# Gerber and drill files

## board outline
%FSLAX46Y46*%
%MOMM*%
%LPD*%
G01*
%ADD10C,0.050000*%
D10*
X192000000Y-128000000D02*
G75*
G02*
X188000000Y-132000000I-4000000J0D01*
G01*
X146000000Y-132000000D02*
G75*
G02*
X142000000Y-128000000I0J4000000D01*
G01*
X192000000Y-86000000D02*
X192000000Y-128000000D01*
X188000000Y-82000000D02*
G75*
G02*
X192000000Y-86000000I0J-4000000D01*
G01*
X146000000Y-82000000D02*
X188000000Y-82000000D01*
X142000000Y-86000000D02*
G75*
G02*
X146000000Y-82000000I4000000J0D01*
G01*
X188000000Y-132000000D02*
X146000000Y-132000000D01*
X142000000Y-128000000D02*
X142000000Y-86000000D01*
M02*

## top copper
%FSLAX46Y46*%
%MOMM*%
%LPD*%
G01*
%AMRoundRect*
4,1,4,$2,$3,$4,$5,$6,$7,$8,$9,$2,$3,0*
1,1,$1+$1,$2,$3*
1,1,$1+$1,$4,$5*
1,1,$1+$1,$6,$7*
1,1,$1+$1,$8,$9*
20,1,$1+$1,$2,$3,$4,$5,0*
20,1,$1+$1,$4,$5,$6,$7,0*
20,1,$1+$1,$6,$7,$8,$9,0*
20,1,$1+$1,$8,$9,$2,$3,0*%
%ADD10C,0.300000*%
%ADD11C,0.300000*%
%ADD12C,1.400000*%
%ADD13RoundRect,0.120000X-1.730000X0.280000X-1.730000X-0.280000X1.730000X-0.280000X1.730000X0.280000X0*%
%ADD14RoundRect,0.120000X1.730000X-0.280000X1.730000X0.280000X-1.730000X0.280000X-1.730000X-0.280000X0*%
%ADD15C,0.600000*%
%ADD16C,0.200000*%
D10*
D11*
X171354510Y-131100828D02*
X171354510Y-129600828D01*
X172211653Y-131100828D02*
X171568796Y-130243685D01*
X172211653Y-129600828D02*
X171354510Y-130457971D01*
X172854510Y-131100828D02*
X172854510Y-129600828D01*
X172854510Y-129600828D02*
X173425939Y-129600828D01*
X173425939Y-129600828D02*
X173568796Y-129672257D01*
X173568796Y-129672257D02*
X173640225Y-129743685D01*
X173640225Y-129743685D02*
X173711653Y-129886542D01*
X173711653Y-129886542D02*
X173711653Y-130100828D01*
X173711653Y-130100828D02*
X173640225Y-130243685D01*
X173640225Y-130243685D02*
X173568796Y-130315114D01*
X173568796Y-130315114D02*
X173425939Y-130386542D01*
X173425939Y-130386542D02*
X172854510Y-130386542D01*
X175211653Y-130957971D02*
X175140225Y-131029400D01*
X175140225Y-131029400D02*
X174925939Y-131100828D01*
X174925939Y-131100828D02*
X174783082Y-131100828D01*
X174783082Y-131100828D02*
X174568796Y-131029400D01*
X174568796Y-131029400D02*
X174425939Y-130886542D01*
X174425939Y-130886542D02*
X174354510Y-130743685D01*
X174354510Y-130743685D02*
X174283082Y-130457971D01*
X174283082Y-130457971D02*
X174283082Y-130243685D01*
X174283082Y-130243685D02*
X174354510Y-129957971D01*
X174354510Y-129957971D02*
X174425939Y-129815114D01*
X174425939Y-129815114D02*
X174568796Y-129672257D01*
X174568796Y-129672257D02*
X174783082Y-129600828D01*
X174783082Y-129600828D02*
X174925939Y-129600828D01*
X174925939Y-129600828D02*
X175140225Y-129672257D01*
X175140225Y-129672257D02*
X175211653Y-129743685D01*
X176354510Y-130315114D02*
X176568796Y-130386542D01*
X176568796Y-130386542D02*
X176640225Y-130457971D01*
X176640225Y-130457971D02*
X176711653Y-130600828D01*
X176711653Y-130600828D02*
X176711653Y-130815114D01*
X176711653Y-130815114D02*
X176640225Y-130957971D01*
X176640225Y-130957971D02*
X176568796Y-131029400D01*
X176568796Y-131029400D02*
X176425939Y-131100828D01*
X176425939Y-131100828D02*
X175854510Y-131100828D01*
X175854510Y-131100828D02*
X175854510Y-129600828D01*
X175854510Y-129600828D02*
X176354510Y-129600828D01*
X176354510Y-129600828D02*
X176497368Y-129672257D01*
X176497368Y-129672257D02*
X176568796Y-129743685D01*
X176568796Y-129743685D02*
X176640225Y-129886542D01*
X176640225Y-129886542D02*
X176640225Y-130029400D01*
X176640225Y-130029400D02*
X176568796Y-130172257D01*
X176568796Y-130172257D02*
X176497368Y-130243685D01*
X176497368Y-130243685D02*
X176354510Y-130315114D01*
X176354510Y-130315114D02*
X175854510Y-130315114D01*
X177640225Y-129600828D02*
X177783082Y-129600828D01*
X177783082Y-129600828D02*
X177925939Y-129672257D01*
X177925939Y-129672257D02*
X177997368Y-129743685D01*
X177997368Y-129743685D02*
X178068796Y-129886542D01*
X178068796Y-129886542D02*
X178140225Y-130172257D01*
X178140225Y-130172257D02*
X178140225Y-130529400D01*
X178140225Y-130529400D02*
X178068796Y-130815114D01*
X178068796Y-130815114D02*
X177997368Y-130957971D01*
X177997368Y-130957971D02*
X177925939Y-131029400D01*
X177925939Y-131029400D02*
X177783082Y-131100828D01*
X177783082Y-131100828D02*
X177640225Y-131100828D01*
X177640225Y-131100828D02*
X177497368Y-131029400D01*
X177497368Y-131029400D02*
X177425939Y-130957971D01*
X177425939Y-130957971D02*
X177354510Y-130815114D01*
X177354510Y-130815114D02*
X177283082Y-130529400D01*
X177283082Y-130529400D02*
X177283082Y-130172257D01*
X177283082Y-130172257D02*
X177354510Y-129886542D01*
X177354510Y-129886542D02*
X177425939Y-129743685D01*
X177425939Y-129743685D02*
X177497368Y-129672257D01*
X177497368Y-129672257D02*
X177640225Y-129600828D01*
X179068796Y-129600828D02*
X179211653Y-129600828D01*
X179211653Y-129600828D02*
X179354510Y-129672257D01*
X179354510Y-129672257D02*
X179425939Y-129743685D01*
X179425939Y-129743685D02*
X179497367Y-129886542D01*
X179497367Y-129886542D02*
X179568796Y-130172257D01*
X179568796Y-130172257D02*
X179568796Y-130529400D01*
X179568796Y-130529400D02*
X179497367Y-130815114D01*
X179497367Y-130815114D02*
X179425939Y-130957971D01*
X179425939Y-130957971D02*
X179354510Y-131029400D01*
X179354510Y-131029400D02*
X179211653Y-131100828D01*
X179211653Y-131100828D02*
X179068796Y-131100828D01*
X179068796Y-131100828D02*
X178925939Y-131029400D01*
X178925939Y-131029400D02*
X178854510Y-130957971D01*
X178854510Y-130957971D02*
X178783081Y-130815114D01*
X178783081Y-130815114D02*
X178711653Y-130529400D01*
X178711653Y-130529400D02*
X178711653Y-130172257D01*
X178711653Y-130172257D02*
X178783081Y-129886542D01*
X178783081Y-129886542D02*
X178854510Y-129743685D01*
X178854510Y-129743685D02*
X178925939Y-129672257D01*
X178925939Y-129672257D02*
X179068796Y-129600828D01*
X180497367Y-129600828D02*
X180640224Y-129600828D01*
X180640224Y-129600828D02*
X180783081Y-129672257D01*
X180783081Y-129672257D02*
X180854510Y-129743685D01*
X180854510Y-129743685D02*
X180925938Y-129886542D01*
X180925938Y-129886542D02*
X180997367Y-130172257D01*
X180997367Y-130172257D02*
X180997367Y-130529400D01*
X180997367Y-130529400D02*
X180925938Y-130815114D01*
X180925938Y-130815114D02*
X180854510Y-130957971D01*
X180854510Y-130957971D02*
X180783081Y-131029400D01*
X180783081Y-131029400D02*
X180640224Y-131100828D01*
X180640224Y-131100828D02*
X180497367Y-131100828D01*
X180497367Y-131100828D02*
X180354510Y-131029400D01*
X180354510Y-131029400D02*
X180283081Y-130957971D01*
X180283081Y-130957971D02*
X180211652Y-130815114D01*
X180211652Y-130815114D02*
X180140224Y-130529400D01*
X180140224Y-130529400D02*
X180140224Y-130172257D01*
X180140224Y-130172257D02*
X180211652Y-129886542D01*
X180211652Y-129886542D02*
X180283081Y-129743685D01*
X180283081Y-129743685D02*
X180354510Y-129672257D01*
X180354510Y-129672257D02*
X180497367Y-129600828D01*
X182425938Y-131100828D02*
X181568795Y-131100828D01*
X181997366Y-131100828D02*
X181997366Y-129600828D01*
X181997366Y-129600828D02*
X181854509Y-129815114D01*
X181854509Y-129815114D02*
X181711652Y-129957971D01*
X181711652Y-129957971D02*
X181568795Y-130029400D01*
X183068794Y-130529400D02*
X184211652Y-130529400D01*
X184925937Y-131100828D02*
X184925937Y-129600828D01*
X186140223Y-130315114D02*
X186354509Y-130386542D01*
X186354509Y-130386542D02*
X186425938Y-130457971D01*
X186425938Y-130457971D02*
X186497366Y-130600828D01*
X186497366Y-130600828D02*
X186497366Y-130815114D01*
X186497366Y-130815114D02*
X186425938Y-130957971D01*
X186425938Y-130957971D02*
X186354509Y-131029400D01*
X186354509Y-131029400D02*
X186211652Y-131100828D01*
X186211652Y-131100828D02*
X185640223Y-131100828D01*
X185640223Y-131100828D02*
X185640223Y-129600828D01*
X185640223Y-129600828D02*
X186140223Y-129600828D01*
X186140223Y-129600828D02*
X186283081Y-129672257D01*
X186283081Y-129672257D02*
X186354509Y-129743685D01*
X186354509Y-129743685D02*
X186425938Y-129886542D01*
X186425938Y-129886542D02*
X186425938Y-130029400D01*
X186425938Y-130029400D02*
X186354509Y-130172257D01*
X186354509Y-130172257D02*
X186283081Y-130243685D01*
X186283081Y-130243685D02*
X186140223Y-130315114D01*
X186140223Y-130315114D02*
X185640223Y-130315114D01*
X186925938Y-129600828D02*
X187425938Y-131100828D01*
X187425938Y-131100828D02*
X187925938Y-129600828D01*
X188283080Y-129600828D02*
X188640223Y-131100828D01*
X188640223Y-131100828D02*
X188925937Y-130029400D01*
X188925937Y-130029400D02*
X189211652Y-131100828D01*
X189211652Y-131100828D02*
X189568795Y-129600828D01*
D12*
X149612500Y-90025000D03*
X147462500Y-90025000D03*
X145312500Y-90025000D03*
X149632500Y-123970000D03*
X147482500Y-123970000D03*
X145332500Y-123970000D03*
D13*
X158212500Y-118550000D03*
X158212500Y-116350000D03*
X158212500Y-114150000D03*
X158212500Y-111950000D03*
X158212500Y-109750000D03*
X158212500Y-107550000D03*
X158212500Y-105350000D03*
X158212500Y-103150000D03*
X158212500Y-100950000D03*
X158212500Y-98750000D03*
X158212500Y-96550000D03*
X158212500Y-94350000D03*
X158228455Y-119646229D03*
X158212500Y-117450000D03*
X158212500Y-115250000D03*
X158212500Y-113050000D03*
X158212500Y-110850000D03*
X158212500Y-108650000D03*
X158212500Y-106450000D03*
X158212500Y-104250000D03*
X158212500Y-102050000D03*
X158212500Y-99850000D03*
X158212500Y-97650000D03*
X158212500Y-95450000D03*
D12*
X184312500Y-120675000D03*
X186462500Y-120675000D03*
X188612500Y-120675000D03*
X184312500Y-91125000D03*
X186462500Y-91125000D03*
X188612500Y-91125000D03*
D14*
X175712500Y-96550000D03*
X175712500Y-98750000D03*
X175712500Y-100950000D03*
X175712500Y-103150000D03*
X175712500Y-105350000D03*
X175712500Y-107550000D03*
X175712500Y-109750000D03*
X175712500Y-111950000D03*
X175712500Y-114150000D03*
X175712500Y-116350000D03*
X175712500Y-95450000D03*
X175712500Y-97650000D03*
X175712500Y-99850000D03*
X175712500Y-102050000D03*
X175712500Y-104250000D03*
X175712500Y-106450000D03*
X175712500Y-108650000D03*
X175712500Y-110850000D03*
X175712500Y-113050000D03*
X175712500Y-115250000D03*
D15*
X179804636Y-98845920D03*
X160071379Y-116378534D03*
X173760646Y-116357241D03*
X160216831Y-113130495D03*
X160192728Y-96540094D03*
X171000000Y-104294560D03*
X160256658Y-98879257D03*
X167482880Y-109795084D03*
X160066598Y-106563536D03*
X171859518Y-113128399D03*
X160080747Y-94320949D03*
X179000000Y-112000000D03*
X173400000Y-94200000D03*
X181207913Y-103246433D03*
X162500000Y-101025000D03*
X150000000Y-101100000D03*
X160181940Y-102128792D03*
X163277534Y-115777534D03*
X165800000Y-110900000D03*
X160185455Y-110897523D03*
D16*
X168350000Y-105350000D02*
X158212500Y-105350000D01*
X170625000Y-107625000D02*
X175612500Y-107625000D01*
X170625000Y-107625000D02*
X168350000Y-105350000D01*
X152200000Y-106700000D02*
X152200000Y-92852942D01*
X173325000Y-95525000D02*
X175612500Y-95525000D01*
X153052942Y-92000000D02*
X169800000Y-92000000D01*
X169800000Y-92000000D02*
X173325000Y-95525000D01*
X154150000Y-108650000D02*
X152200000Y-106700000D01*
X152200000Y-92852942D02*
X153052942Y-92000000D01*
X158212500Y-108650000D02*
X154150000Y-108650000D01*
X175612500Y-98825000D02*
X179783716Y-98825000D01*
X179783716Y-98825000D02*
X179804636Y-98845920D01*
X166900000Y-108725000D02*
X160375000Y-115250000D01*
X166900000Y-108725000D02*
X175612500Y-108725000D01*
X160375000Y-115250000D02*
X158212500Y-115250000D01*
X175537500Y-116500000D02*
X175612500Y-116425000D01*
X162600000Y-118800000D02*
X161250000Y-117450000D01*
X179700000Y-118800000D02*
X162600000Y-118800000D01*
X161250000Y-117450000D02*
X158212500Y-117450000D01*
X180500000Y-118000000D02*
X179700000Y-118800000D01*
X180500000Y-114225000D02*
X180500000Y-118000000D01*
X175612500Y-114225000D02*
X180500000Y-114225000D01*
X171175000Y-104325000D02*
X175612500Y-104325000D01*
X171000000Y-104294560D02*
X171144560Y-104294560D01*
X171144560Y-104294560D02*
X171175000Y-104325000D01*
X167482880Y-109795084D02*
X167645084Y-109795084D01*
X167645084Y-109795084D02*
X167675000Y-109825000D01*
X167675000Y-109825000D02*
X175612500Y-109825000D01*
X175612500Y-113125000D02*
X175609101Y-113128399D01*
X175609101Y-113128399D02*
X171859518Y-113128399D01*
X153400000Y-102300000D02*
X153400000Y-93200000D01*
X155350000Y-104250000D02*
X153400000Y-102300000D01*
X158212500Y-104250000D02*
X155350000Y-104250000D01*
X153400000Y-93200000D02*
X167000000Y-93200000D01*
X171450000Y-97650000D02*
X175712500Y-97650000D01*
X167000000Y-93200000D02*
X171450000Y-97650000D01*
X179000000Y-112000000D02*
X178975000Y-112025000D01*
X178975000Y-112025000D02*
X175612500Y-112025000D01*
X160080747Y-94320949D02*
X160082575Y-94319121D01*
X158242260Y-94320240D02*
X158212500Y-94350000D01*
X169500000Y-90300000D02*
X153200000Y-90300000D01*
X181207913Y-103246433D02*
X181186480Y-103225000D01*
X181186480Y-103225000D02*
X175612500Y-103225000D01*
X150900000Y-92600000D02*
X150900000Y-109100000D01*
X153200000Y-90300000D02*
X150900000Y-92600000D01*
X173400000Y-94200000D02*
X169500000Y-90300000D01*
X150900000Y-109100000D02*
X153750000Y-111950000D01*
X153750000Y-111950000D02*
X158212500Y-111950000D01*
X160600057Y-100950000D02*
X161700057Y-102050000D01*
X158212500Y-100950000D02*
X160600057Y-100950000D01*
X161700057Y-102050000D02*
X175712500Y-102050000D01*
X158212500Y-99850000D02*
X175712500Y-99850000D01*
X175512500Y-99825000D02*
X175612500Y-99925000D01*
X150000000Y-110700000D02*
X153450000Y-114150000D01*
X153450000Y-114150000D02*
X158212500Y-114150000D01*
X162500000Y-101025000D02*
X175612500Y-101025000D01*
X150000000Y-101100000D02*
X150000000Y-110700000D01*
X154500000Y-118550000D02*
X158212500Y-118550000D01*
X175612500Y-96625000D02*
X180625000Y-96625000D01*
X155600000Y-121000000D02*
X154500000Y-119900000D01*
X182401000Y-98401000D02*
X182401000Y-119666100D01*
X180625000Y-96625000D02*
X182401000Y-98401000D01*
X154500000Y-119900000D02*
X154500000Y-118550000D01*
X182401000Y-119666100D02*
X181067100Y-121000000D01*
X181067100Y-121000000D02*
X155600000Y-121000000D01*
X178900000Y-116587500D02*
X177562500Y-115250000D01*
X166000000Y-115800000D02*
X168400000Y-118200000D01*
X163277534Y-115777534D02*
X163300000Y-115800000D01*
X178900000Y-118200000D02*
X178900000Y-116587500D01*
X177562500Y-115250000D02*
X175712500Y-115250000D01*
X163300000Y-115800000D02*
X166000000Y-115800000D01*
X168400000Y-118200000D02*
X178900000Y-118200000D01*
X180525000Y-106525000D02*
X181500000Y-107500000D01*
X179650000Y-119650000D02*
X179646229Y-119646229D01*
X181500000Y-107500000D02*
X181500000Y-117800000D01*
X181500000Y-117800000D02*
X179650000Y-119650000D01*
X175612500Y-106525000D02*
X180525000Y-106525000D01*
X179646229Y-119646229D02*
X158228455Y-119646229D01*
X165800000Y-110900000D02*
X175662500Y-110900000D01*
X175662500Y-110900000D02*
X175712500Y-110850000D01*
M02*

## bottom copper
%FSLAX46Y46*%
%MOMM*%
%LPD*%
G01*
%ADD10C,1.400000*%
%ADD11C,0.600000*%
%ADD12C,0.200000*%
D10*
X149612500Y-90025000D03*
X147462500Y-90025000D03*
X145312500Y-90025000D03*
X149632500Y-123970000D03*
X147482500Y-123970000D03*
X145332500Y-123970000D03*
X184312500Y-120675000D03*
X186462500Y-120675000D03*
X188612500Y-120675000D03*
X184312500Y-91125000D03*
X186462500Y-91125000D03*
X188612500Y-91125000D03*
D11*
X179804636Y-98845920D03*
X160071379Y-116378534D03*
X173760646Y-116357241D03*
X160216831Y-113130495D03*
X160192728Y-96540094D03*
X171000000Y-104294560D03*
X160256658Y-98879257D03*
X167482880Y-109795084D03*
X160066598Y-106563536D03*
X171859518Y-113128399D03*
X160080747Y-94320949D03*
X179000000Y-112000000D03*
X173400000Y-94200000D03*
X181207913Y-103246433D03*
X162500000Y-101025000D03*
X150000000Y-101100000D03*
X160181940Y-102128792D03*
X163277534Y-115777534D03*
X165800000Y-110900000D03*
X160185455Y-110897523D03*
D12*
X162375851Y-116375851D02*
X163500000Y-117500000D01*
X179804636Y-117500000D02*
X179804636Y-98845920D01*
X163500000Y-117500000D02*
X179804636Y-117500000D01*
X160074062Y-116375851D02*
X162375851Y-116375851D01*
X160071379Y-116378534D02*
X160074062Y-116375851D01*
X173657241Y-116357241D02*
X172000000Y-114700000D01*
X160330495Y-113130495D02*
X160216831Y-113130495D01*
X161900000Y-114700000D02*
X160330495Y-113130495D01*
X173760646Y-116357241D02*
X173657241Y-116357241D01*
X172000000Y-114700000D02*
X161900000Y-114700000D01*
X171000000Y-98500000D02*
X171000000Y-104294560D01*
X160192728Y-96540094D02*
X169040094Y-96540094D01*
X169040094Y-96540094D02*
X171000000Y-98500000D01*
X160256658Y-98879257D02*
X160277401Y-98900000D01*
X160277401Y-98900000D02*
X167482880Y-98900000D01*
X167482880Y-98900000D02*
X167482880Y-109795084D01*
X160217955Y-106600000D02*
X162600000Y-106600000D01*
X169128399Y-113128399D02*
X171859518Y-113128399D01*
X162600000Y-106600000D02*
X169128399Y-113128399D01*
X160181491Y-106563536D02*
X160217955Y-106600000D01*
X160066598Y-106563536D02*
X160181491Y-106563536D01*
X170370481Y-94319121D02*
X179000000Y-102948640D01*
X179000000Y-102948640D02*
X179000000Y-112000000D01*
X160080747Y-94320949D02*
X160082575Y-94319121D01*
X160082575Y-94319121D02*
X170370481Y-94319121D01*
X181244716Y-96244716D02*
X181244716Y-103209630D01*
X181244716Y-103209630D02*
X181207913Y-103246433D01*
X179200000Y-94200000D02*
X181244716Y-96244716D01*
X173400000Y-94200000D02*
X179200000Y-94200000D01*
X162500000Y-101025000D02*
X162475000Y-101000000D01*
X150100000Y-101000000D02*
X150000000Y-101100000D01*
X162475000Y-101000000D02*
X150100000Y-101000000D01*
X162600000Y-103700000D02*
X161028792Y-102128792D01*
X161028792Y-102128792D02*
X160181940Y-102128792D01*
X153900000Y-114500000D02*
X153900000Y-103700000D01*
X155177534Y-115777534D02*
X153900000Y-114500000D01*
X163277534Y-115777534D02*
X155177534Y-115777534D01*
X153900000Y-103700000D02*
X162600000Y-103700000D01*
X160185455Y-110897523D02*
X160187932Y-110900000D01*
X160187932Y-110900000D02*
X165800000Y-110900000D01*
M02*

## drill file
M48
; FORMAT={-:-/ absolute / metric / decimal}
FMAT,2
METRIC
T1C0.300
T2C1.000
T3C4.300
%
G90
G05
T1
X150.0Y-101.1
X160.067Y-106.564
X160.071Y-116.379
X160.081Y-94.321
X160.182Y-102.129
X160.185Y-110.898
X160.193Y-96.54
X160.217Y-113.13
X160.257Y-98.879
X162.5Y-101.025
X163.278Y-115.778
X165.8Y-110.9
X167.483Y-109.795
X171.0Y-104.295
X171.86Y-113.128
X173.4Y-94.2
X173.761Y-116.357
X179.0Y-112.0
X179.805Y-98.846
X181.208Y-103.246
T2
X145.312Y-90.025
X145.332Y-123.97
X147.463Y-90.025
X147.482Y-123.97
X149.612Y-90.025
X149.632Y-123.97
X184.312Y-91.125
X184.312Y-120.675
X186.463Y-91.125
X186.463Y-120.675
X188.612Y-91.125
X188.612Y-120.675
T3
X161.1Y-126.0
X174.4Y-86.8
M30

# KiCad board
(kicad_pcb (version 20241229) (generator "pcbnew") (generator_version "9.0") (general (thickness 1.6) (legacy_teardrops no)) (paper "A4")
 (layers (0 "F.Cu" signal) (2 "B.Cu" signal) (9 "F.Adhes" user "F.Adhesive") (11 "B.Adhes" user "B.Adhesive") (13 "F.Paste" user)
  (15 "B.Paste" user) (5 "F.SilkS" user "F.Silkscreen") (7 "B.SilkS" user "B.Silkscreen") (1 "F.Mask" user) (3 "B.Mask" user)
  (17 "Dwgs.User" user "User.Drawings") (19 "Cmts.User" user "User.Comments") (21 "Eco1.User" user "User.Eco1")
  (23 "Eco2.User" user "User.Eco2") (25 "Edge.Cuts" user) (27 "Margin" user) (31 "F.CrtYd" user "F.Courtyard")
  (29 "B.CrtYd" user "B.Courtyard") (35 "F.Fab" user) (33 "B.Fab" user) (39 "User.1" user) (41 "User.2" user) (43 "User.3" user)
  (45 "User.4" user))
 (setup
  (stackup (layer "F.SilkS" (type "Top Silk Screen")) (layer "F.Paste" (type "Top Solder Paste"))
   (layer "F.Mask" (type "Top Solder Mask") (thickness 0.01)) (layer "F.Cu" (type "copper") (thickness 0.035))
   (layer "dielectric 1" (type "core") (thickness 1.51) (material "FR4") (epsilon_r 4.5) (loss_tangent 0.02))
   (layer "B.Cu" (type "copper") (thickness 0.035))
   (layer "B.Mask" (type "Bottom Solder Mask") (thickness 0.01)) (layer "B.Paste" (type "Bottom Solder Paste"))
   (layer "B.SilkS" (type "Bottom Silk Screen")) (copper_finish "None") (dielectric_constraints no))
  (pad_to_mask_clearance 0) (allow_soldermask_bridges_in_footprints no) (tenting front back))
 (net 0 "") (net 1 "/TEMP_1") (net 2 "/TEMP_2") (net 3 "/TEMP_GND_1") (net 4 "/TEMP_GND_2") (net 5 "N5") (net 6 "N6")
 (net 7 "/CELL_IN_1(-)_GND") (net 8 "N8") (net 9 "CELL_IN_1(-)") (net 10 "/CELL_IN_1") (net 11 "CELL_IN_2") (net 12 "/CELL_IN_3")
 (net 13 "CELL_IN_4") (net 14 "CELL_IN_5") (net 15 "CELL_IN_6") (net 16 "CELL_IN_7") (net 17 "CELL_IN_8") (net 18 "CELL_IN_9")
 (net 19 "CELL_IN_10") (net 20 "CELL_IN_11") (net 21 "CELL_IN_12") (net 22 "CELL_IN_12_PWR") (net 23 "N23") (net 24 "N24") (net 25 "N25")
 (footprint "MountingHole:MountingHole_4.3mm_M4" (layer "F.Cu") (at 174.4 86.8)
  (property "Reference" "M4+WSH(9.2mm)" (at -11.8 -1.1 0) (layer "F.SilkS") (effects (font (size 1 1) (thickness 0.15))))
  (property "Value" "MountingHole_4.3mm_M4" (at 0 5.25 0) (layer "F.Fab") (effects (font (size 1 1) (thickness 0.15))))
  (pad "" np_thru_hole circle (at 0 0) (size 4.3 4.3) (drill 4.3) (layers "*.Cu" "*.Mask")))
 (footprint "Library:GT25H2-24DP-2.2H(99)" (layer "F.Cu") (at 160.4625 107 -90)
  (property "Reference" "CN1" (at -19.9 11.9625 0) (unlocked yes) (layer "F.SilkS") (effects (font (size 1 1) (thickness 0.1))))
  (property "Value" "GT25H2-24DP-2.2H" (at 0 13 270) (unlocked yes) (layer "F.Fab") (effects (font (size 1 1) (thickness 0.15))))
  (pad "" np_thru_hole circle (at -16.975 10.85 270) (size 1.4 1.4) (drill 1) (layers "*.Cu" "*.Mask"))
  (pad "" np_thru_hole circle (at -16.975 13 270) (size 1.4 1.4) (drill 1) (layers "*.Cu" "*.Mask"))
  (pad "" np_thru_hole circle (at -16.975 15.15 270) (size 1.4 1.4) (drill 1) (layers "*.Cu" "*.Mask"))
  (pad "" np_thru_hole circle (at 16.97 10.83 270) (size 1.4 1.4) (drill 1) (layers "*.Cu" "*.Mask"))
  (pad "" np_thru_hole circle (at 16.97 12.98 270) (size 1.4 1.4) (drill 1) (layers "*.Cu" "*.Mask"))
  (pad "" np_thru_hole circle (at 16.97 15.13 270) (size 1.4 1.4) (drill 1) (layers "*.Cu" "*.Mask"))
  (pad "1" smd roundrect (at 11.55 2.25 270) (size 0.8 3.7) (layers "F.Cu" "F.Mask" "F.Paste") (roundrect_rratio 0.15) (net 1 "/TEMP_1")
   (thermal_bridge_angle 45))
  (pad "2" smd roundrect (at 9.35 2.25 270) (size 0.8 3.7) (layers "F.Cu" "F.Mask" "F.Paste") (roundrect_rratio 0.15) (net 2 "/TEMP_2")
   (thermal_bridge_angle 45))
  (pad "3" smd roundrect (at 7.15 2.25 270) (size 0.8 3.7) (layers "F.Cu" "F.Mask" "F.Paste") (roundrect_rratio 0.15) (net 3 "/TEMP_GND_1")
   (thermal_bridge_angle 45))
  (pad "4" smd roundrect (at 4.95 2.25 270) (size 0.8 3.7) (layers "F.Cu" "F.Mask" "F.Paste") (roundrect_rratio 0.15) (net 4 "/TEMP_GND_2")
   (thermal_bridge_angle 45))
  (pad "5" smd roundrect (at 2.75 2.25 270) (size 0.8 3.7) (layers "F.Cu" "F.Mask" "F.Paste") (roundrect_rratio 0.15) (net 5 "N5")
   (thermal_bridge_angle 45))
  (pad "6" smd roundrect (at 0.55 2.25 270) (size 0.8 3.7) (layers "F.Cu" "F.Mask" "F.Paste") (roundrect_rratio 0.15) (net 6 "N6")
   (thermal_bridge_angle 45))
  (pad "7" smd roundrect (at -1.65 2.25 270) (size 0.8 3.7) (layers "F.Cu" "F.Mask" "F.Paste") (roundrect_rratio 0.15)
   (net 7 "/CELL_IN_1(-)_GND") (thermal_bridge_angle 45))
  (pad "8" smd roundrect (at -3.85 2.25 270) (size 0.8 3.7) (layers "F.Cu" "F.Mask" "F.Paste") (roundrect_rratio 0.15) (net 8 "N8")
   (thermal_bridge_angle 45))
  (pad "9" smd roundrect (at -6.05 2.25 270) (size 0.8 3.7) (layers "F.Cu" "F.Mask" "F.Paste") (roundrect_rratio 0.15)
   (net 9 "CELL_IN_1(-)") (thermal_bridge_angle 45))
  (pad "10" smd roundrect (at -8.25 2.25 270) (size 0.8 3.7) (layers "F.Cu" "F.Mask" "F.Paste") (roundrect_rratio 0.15)
   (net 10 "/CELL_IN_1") (thermal_bridge_angle 45))
  (pad "11" smd roundrect (at -10.45 2.25 270) (size 0.8 3.7) (layers "F.Cu" "F.Mask" "F.Paste") (roundrect_rratio 0.15)
   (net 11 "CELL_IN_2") (thermal_bridge_angle 45))
  (pad "12" smd roundrect (at -12.65 2.25 270) (size 0.8 3.7) (layers "F.Cu" "F.Mask" "F.Paste") (roundrect_rratio 0.15)
   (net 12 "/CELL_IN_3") (thermal_bridge_angle 45))
  (pad "13" smd roundrect (at 12.646229 2.234045 270) (size 0.8 3.7) (layers "F.Cu" "F.Mask" "F.Paste") (roundrect_rratio 0.15)
   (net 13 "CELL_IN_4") (thermal_bridge_angle 45))
  (pad "14" smd roundrect (at 10.45 2.25 270) (size 0.8 3.7) (layers "F.Cu" "F.Mask" "F.Paste") (roundrect_rratio 0.15) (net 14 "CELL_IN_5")
   (thermal_bridge_angle 45))
  (pad "15" smd roundrect (at 8.25 2.25 270) (size 0.8 3.7) (layers "F.Cu" "F.Mask" "F.Paste") (roundrect_rratio 0.15) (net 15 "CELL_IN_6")
   (thermal_bridge_angle 45))
  (pad "16" smd roundrect (at 6.05 2.25 270) (size 0.8 3.7) (layers "F.Cu" "F.Mask" "F.Paste") (roundrect_rratio 0.15) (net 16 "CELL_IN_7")
   (thermal_bridge_angle 45))
  (pad "17" smd roundrect (at 3.85 2.25 270) (size 0.8 3.7) (layers "F.Cu" "F.Mask" "F.Paste") (roundrect_rratio 0.15) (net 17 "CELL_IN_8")
   (thermal_bridge_angle 45))
  (pad "18" smd roundrect (at 1.65 2.25 270) (size 0.8 3.7) (layers "F.Cu" "F.Mask" "F.Paste") (roundrect_rratio 0.15) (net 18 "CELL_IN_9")
   (thermal_bridge_angle 45))
  (pad "19" smd roundrect (at -0.55 2.25 270) (size 0.8 3.7) (layers "F.Cu" "F.Mask" "F.Paste") (roundrect_rratio 0.15)
   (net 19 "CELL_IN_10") (thermal_bridge_angle 45))
  (pad "20" smd roundrect (at -2.75 2.25 270) (size 0.8 3.7) (layers "F.Cu" "F.Mask" "F.Paste") (roundrect_rratio 0.15)
   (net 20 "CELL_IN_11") (thermal_bridge_angle 45))
  (pad "21" smd roundrect (at -4.95 2.25 270) (size 0.8 3.7) (layers "F.Cu" "F.Mask" "F.Paste") (roundrect_rratio 0.15)
   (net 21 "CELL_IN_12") (thermal_bridge_angle 45))
  (pad "22" smd roundrect (at -7.15 2.25 270) (size 0.8 3.7) (layers "F.Cu" "F.Mask" "F.Paste") (roundrect_rratio 0.15)
   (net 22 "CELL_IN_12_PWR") (thermal_bridge_angle 45))
  (pad "23" smd roundrect (at -9.35 2.25 270) (size 0.8 3.7) (layers "F.Cu" "F.Mask" "F.Paste") (roundrect_rratio 0.15) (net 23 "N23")
   (thermal_bridge_angle 45))
  (pad "24" smd roundrect (at -11.55 2.25 270) (size 0.8 3.7) (layers "F.Cu" "F.Mask" "F.Paste") (roundrect_rratio 0.15) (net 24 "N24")
   (thermal_bridge_angle 45)))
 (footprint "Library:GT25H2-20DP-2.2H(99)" (layer "F.Cu") (at 173.4625 105.9 90)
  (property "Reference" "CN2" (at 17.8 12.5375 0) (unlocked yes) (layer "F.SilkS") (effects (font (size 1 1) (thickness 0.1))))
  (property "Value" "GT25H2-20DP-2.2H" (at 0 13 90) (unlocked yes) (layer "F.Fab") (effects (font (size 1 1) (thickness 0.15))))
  (pad "" np_thru_hole circle (at -14.775 10.85 90) (size 1.4 1.4) (drill 1) (layers "*.Cu" "*.Mask"))
  (pad "" np_thru_hole circle (at -14.775 13 90) (size 1.4 1.4) (drill 1) (layers "*.Cu" "*.Mask"))
  (pad "" np_thru_hole circle (at -14.775 15.15 90) (size 1.4 1.4) (drill 1) (layers "*.Cu" "*.Mask"))
  (pad "" np_thru_hole circle (at 14.775 10.85 90) (size 1.4 1.4) (drill 1) (layers "*.Cu" "*.Mask"))
  (pad "" np_thru_hole circle (at 14.775 13 90) (size 1.4 1.4) (drill 1) (layers "*.Cu" "*.Mask"))
  (pad "" np_thru_hole circle (at 14.775 15.15 90) (size 1.4 1.4) (drill 1) (layers "*.Cu" "*.Mask"))
  (pad "1" smd roundrect (at 9.35 2.25 90) (size 0.8 3.7) (layers "F.Cu" "F.Mask" "F.Paste") (roundrect_rratio 0.15) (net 1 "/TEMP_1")
   (thermal_bridge_angle 45))
  (pad "2" smd roundrect (at 7.15 2.25 90) (size 0.8 3.7) (layers "F.Cu" "F.Mask" "F.Paste") (roundrect_rratio 0.15) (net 2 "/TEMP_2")
   (thermal_bridge_angle 45))
  (pad "3" smd roundrect (at 4.95 2.25 90) (size 0.8 3.7) (layers "F.Cu" "F.Mask" "F.Paste") (roundrect_rratio 0.15) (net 3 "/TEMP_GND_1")
   (thermal_bridge_angle 45))
  (pad "4" smd roundrect (at 2.75 2.25 90) (size 0.8 3.7) (layers "F.Cu" "F.Mask" "F.Paste") (roundrect_rratio 0.15) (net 4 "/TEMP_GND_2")
   (thermal_bridge_angle 45))
  (pad "5" smd roundrect (at 0.55 2.25 90) (size 0.8 3.7) (layers "F.Cu" "F.Mask" "F.Paste") (roundrect_rratio 0.15) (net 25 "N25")
   (thermal_bridge_angle 45))
  (pad "6" smd roundrect (at -1.65 2.25 90) (size 0.8 3.7) (layers "F.Cu" "F.Mask" "F.Paste") (roundrect_rratio 0.15)
   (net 7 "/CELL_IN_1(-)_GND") (thermal_bridge_angle 45))
  (pad "7" smd roundrect (at -3.85 2.25 90) (size 0.8 3.7) (layers "F.Cu" "F.Mask" "F.Paste") (roundrect_rratio 0.15) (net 10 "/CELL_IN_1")
   (thermal_bridge_angle 45))
  (pad "8" smd roundrect (at -6.05 2.25 90) (size 0.8 3.7) (layers "F.Cu" "F.Mask" "F.Paste") (roundrect_rratio 0.15) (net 12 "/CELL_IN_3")
   (thermal_bridge_angle 45))
  (pad "9" smd roundrect (at -8.25 2.25 90) (size 0.8 3.7) (layers "F.Cu" "F.Mask" "F.Paste") (roundrect_rratio 0.15) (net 14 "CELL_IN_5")
   (thermal_bridge_angle 45))
  (pad "10" smd roundrect (at -10.45 2.25 90) (size 0.8 3.7) (layers "F.Cu" "F.Mask" "F.Paste") (roundrect_rratio 0.15) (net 16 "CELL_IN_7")
   (thermal_bridge_angle 45))
  (pad "11" smd roundrect (at 10.45 2.25 90) (size 0.8 3.7) (layers "F.Cu" "F.Mask" "F.Paste") (roundrect_rratio 0.15) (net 18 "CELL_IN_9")
   (thermal_bridge_angle 45))
  (pad "12" smd roundrect (at 8.25 2.25 90) (size 0.8 3.7) (layers "F.Cu" "F.Mask" "F.Paste") (roundrect_rratio 0.15) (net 20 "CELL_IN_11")
   (thermal_bridge_angle 45))
  (pad "13" smd roundrect (at 6.05 2.25 90) (size 0.8 3.7) (layers "F.Cu" "F.Mask" "F.Paste") (roundrect_rratio 0.15)
   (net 22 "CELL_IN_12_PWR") (thermal_bridge_angle 45))
  (pad "14" smd roundrect (at 3.85 2.25 90) (size 0.8 3.7) (layers "F.Cu" "F.Mask" "F.Paste") (roundrect_rratio 0.15) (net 9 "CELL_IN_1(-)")
   (thermal_bridge_angle 45))
  (pad "15" smd roundrect (at 1.65 2.25 90) (size 0.8 3.7) (layers "F.Cu" "F.Mask" "F.Paste") (roundrect_rratio 0.15) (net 11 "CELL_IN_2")
   (thermal_bridge_angle 45))
  (pad "16" smd roundrect (at -0.55 2.25 90) (size 0.8 3.7) (layers "F.Cu" "F.Mask" "F.Paste") (roundrect_rratio 0.15) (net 13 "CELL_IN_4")
   (thermal_bridge_angle 45))
  (pad "17" smd roundrect (at -2.75 2.25 90) (size 0.8 3.7) (layers "F.Cu" "F.Mask" "F.Paste") (roundrect_rratio 0.15) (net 15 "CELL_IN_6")
   (thermal_bridge_angle 45))
  (pad "18" smd roundrect (at -4.95 2.25 90) (size 0.8 3.7) (layers "F.Cu" "F.Mask" "F.Paste") (roundrect_rratio 0.15) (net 17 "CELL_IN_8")
   (thermal_bridge_angle 45))
  (pad "19" smd roundrect (at -7.15 2.25 90) (size 0.8 3.7) (layers "F.Cu" "F.Mask" "F.Paste") (roundrect_rratio 0.15) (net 19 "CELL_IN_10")
   (thermal_bridge_angle 45))
  (pad "20" smd roundrect (at -9.35 2.25 90) (size 0.8 3.7) (layers "F.Cu" "F.Mask" "F.Paste") (roundrect_rratio 0.15) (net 21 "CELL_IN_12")
   (thermal_bridge_angle 45)))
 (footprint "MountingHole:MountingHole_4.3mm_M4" (layer "F.Cu") (at 161.1 126)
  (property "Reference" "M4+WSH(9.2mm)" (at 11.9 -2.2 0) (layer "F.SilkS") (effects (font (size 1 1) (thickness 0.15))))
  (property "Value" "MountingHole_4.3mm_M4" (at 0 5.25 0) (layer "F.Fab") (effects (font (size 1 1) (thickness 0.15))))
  (pad "" np_thru_hole circle (at 0 0) (size 4.3 4.3) (drill 4.3) (layers "*.Cu" "*.Mask")))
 (gr_arc (start 192 128) (mid 190.828427 130.828427) (end 188 132) (stroke (width 0.05) (type default)) (layer "Edge.Cuts"))
 (gr_arc (start 146 132) (mid 143.171573 130.828427) (end 142 128) (stroke (width 0.05) (type default)) (layer "Edge.Cuts"))
 (gr_line (start 192 86) (end 192 128) (stroke (width 0.05) (type default)) (layer "Edge.Cuts"))
 (gr_arc (start 188 82) (mid 190.828427 83.171573) (end 192 86) (stroke (width 0.05) (type default)) (layer "Edge.Cuts"))
 (gr_line (start 146 82) (end 188 82) (stroke (width 0.05) (type default)) (layer "Edge.Cuts"))
 (gr_arc (start 142 86) (mid 143.171573 83.171573) (end 146 82) (stroke (width 0.05) (type default)) (layer "Edge.Cuts"))
 (gr_line (start 188 132) (end 146 132) (stroke (width 0.05) (type default)) (layer "Edge.Cuts"))
 (gr_line (start 142 128) (end 142 86) (stroke (width 0.05) (type default)) (layer "Edge.Cuts"))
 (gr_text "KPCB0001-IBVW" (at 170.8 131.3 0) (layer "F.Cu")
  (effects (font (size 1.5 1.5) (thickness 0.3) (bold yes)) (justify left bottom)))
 (segment (start 168.35 105.35) (end 158.2125 105.35) (width 0.2) (layer "F.Cu") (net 7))
 (segment (start 170.625 107.625) (end 175.6125 107.625) (width 0.2) (layer "F.Cu") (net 7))
 (segment (start 170.625 107.625) (end 168.35 105.35) (width 0.2) (layer "F.Cu") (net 7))
 (segment (start 152.2 106.7) (end 152.2 92.852942) (width 0.2) (layer "F.Cu") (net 18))
 (segment (start 173.325 95.525) (end 175.6125 95.525) (width 0.2) (layer "F.Cu") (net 18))
 (segment (start 153.052942 92) (end 169.8 92) (width 0.2) (layer "F.Cu") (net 18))
 (segment (start 169.8 92) (end 173.325 95.525) (width 0.2) (layer "F.Cu") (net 18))
 (segment (start 154.15 108.65) (end 152.2 106.7) (width 0.2) (layer "F.Cu") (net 18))
 (segment (start 152.2 92.852942) (end 153.052942 92) (width 0.2) (layer "F.Cu") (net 18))
 (segment (start 158.2125 108.65) (end 154.15 108.65) (width 0.2) (layer "F.Cu") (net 18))
 (segment (start 175.6125 98.825) (end 179.783716 98.825) (width 0.2) (layer "F.Cu") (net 2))
 (segment (start 179.783716 98.825) (end 179.804636 98.84592) (width 0.2) (layer "F.Cu") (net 2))
 (via (at 179.804636 98.84592) (size 0.6) (drill 0.3) (layers "F.Cu" "B.Cu") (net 2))
 (via (at 160.071379 116.378534) (size 0.6) (drill 0.3) (layers "F.Cu" "B.Cu") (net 2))
 (segment (start 162.375851 116.375851) (end 163.5 117.5) (width 0.2) (layer "B.Cu") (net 2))
 (segment (start 179.804636 117.5) (end 179.804636 98.84592) (width 0.2) (layer "B.Cu") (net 2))
 (segment (start 163.5 117.5) (end 179.804636 117.5) (width 0.2) (layer "B.Cu") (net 2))
 (segment (start 160.074062 116.375851) (end 162.375851 116.375851) (width 0.2) (layer "B.Cu") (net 2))
 (segment (start 160.071379 116.378534) (end 160.074062 116.375851) (width 0.2) (layer "B.Cu") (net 2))
 (segment (start 166.9 108.725) (end 160.375 115.25) (width 0.2) (layer "F.Cu") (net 15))
 (segment (start 166.9 108.725) (end 175.6125 108.725) (width 0.2) (layer "F.Cu") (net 15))
 (segment (start 160.375 115.25) (end 158.2125 115.25) (width 0.2) (layer "F.Cu") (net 15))
 (segment (start 175.5375 116.5) (end 175.6125 116.425) (width 0.2) (layer "F.Cu") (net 16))
 (via (at 173.760646 116.357241) (size 0.6) (drill 0.3) (layers "F.Cu" "B.Cu") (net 16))
 (via (at 160.216831 113.130495) (size 0.6) (drill 0.3) (layers "F.Cu" "B.Cu") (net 16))
 (segment (start 173.657241 116.357241) (end 172 114.7) (width 0.2) (layer "B.Cu") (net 16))
 (segment (start 160.330495 113.130495) (end 160.216831 113.130495) (width 0.2) (layer "B.Cu") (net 16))
 (segment (start 161.9 114.7) (end 160.330495 113.130495) (width 0.2) (layer "B.Cu") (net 16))
 (segment (start 173.760646 116.357241) (end 173.657241 116.357241) (width 0.2) (layer "B.Cu") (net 16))
 (segment (start 172 114.7) (end 161.9 114.7) (width 0.2) (layer "B.Cu") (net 16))
 (segment (start 162.6 118.8) (end 161.25 117.45) (width 0.2) (layer "F.Cu") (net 14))
 (segment (start 179.7 118.8) (end 162.6 118.8) (width 0.2) (layer "F.Cu") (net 14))
 (segment (start 161.25 117.45) (end 158.2125 117.45) (width 0.2) (layer "F.Cu") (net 14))
 (segment (start 180.5 118) (end 179.7 118.8) (width 0.2) (layer "F.Cu") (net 14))
 (segment (start 180.5 114.225) (end 180.5 118) (width 0.2) (layer "F.Cu") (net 14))
 (segment (start 175.6125 114.225) (end 180.5 114.225) (width 0.2) (layer "F.Cu") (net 14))
 (segment (start 171.175 104.325) (end 175.6125 104.325) (width 0.2) (layer "F.Cu") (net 11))
 (segment (start 171 104.29456) (end 171.14456 104.29456) (width 0.2) (layer "F.Cu") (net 11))
 (segment (start 171.14456 104.29456) (end 171.175 104.325) (width 0.2) (layer "F.Cu") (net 11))
 (via (at 160.192728 96.540094) (size 0.6) (drill 0.3) (layers "F.Cu" "B.Cu") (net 11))
 (via (at 171 104.29456) (size 0.6) (drill 0.3) (layers "F.Cu" "B.Cu") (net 11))
 (segment (start 171 98.5) (end 171 104.29456) (width 0.2) (layer "B.Cu") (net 11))
 (segment (start 160.192728 96.540094) (end 169.040094 96.540094) (width 0.2) (layer "B.Cu") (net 11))
 (segment (start 169.040094 96.540094) (end 171 98.5) (width 0.2) (layer "B.Cu") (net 11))
 (segment (start 167.48288 109.795084) (end 167.645084 109.795084) (width 0.2) (layer "F.Cu") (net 10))
 (segment (start 167.645084 109.795084) (end 167.675 109.825) (width 0.2) (layer "F.Cu") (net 10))
 (segment (start 167.675 109.825) (end 175.6125 109.825) (width 0.2) (layer "F.Cu") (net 10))
 (via (at 160.256658 98.879257) (size 0.6) (drill 0.3) (layers "F.Cu" "B.Cu") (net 10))
 (via (at 167.48288 109.795084) (size 0.6) (drill 0.3) (layers "F.Cu" "B.Cu") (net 10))
 (segment (start 160.256658 98.879257) (end 160.277401 98.9) (width 0.2) (layer "B.Cu") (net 10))
 (segment (start 160.277401 98.9) (end 167.48288 98.9) (width 0.2) (layer "B.Cu") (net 10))
 (segment (start 167.48288 98.9) (end 167.48288 109.795084) (width 0.2) (layer "B.Cu") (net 10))
 (segment (start 175.6125 113.125) (end 175.609101 113.128399) (width 0.2) (layer "F.Cu") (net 19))
 (segment (start 175.609101 113.128399) (end 171.859518 113.128399) (width 0.2) (layer "F.Cu") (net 19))
 (via (at 160.066598 106.563536) (size 0.6) (drill 0.3) (layers "F.Cu" "B.Cu") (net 19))
 (via (at 171.859518 113.128399) (size 0.6) (drill 0.3) (layers "F.Cu" "B.Cu") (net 19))
 (segment (start 160.217955 106.6) (end 162.6 106.6) (width 0.2) (layer "B.Cu") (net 19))
 (segment (start 169.128399 113.128399) (end 171.859518 113.128399) (width 0.2) (layer "B.Cu") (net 19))
 (segment (start 162.6 106.6) (end 169.128399 113.128399) (width 0.2) (layer "B.Cu") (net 19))
 (segment (start 160.181491 106.563536) (end 160.217955 106.6) (width 0.2) (layer "B.Cu") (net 19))
 (segment (start 160.066598 106.563536) (end 160.181491 106.563536) (width 0.2) (layer "B.Cu") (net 19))
 (segment (start 153.4 102.3) (end 153.4 93.2) (width 0.2) (layer "F.Cu") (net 20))
 (segment (start 155.35 104.25) (end 153.4 102.3) (width 0.2) (layer "F.Cu") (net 20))
 (segment (start 158.2125 104.25) (end 155.35 104.25) (width 0.2) (layer "F.Cu") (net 20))
 (segment (start 153.4 93.2) (end 167 93.2) (width 0.2) (layer "F.Cu") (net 20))
 (segment (start 171.45 97.65) (end 175.7125 97.65) (width 0.2) (layer "F.Cu") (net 20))
 (segment (start 167 93.2) (end 171.45 97.65) (width 0.2) (layer "F.Cu") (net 20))
 (segment (start 179 112) (end 178.975 112.025) (width 0.2) (layer "F.Cu") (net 12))
 (segment (start 178.975 112.025) (end 175.6125 112.025) (width 0.2) (layer "F.Cu") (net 12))
 (segment (start 160.080747 94.320949) (end 160.082575 94.319121) (width 0.2) (layer "F.Cu") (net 12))
 (segment (start 158.24226 94.32024) (end 158.2125 94.35) (width 0.2) (layer "F.Cu") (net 12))
 (via (at 160.080747 94.320949) (size 0.6) (drill 0.3) (layers "F.Cu" "B.Cu") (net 12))
 (via (at 179 112) (size 0.6) (drill 0.3) (layers "F.Cu" "B.Cu") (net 12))
 (segment (start 170.370481 94.319121) (end 179 102.94864) (width 0.2) (layer "B.Cu") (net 12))
 (segment (start 179 102.94864) (end 179 112) (width 0.2) (layer "B.Cu") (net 12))
 (segment (start 160.080747 94.320949) (end 160.082575 94.319121) (width 0.2) (layer "B.Cu") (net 12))
 (segment (start 160.082575 94.319121) (end 170.370481 94.319121) (width 0.2) (layer "B.Cu") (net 12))
 (segment (start 169.5 90.3) (end 153.2 90.3) (width 0.2) (layer "F.Cu") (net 4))
 (segment (start 181.207913 103.246433) (end 181.18648 103.225) (width 0.2) (layer "F.Cu") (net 4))
 (segment (start 181.18648 103.225) (end 175.6125 103.225) (width 0.2) (layer "F.Cu") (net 4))
 (segment (start 150.9 92.6) (end 150.9 109.1) (width 0.2) (layer "F.Cu") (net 4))
 (segment (start 153.2 90.3) (end 150.9 92.6) (width 0.2) (layer "F.Cu") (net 4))
 (segment (start 173.4 94.2) (end 169.5 90.3) (width 0.2) (layer "F.Cu") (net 4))
 (segment (start 150.9 109.1) (end 153.75 111.95) (width 0.2) (layer "F.Cu") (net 4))
 (segment (start 153.75 111.95) (end 158.2125 111.95) (width 0.2) (layer "F.Cu") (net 4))
 (via (at 173.4 94.2) (size 0.6) (drill 0.3) (layers "F.Cu" "B.Cu") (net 4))
 (via (at 181.207913 103.246433) (size 0.6) (drill 0.3) (layers "F.Cu" "B.Cu") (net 4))
 (segment (start 181.244716 96.244716) (end 181.244716 103.20963) (width 0.2) (layer "B.Cu") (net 4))
 (segment (start 181.244716 103.20963) (end 181.207913 103.246433) (width 0.2) (layer "B.Cu") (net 4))
 (segment (start 179.2 94.2) (end 181.244716 96.244716) (width 0.2) (layer "B.Cu") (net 4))
 (segment (start 173.4 94.2) (end 179.2 94.2) (width 0.2) (layer "B.Cu") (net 4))
 (segment (start 160.600057 100.95) (end 161.700057 102.05) (width 0.2) (layer "F.Cu") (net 9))
 (segment (start 158.2125 100.95) (end 160.600057 100.95) (width 0.2) (layer "F.Cu") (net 9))
 (segment (start 161.700057 102.05) (end 175.7125 102.05) (width 0.2) (layer "F.Cu") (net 9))
 (segment (start 158.2125 99.85) (end 175.7125 99.85) (width 0.2) (layer "F.Cu") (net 22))
 (segment (start 175.5125 99.825) (end 175.6125 99.925) (width 0.2) (layer "F.Cu") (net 22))
 (segment (start 150 110.7) (end 153.45 114.15) (width 0.2) (layer "F.Cu") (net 3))
 (segment (start 153.45 114.15) (end 158.2125 114.15) (width 0.2) (layer "F.Cu") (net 3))
 (segment (start 162.5 101.025) (end 175.6125 101.025) (width 0.2) (layer "F.Cu") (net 3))
 (segment (start 150 101.1) (end 150 110.7) (width 0.2) (layer "F.Cu") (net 3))
 (via (at 162.5 101.025) (size 0.6) (drill 0.3) (layers "F.Cu" "B.Cu") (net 3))
 (via (at 150 101.1) (size 0.6) (drill 0.3) (layers "F.Cu" "B.Cu") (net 3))
 (segment (start 162.5 101.025) (end 162.475 101) (width 0.2) (layer "B.Cu") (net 3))
 (segment (start 150.1 101) (end 150 101.1) (width 0.2) (layer "B.Cu") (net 3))
 (segment (start 162.475 101) (end 150.1 101) (width 0.2) (layer "B.Cu") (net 3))
 (segment (start 154.5 118.55) (end 158.2125 118.55) (width 0.2) (layer "F.Cu") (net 1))
 (segment (start 175.6125 96.625) (end 180.625 96.625) (width 0.2) (layer "F.Cu") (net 1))
 (segment (start 155.6 121) (end 154.5 119.9) (width 0.2) (layer "F.Cu") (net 1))
 (segment (start 182.401 98.401) (end 182.401 119.6661) (width 0.2) (layer "F.Cu") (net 1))
 (segment (start 180.625 96.625) (end 182.401 98.401) (width 0.2) (layer "F.Cu") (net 1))
 (segment (start 154.5 119.9) (end 154.5 118.55) (width 0.2) (layer "F.Cu") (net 1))
 (segment (start 182.401 119.6661) (end 181.0671 121) (width 0.2) (layer "F.Cu") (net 1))
 (segment (start 181.0671 121) (end 155.6 121) (width 0.2) (layer "F.Cu") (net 1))
 (segment (start 178.9 116.5875) (end 177.5625 115.25) (width 0.2) (layer "F.Cu") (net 21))
 (segment (start 166 115.8) (end 168.4 118.2) (width 0.2) (layer "F.Cu") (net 21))
 (segment (start 163.277534 115.777534) (end 163.3 115.8) (width 0.2) (layer "F.Cu") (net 21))
 (segment (start 178.9 118.2) (end 178.9 116.5875) (width 0.2) (layer "F.Cu") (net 21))
 (segment (start 177.5625 115.25) (end 175.7125 115.25) (width 0.2) (layer "F.Cu") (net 21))
 (segment (start 163.3 115.8) (end 166 115.8) (width 0.2) (layer "F.Cu") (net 21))
 (segment (start 168.4 118.2) (end 178.9 118.2) (width 0.2) (layer "F.Cu") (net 21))
 (via (at 160.18194 102.128792) (size 0.6) (drill 0.3) (layers "F.Cu" "B.Cu") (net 21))
 (via (at 163.277534 115.777534) (size 0.6) (drill 0.3) (layers "F.Cu" "B.Cu") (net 21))
 (segment (start 162.6 103.7) (end 161.028792 102.128792) (width 0.2) (layer "B.Cu") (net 21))
 (segment (start 161.028792 102.128792) (end 160.18194 102.128792) (width 0.2) (layer "B.Cu") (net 21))
 (segment (start 153.9 114.5) (end 153.9 103.7) (width 0.2) (layer "B.Cu") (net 21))
 (segment (start 155.177534 115.777534) (end 153.9 114.5) (width 0.2) (layer "B.Cu") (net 21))
 (segment (start 163.277534 115.777534) (end 155.177534 115.777534) (width 0.2) (layer "B.Cu") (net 21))
 (segment (start 153.9 103.7) (end 162.6 103.7) (width 0.2) (layer "B.Cu") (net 21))
 (segment (start 180.525 106.525) (end 181.5 107.5) (width 0.2) (layer "F.Cu") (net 13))
 (segment (start 179.65 119.65) (end 179.646229 119.646229) (width 0.2) (layer "F.Cu") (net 13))
 (segment (start 181.5 107.5) (end 181.5 117.8) (width 0.2) (layer "F.Cu") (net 13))
 (segment (start 181.5 117.8) (end 179.65 119.65) (width 0.2) (layer "F.Cu") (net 13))
 (segment (start 175.6125 106.525) (end 180.525 106.525) (width 0.2) (layer "F.Cu") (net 13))
 (segment (start 179.646229 119.646229) (end 158.228455 119.646229) (width 0.2) (layer "F.Cu") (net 13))
 (segment (start 165.8 110.9) (end 175.6625 110.9) (width 0.2) (layer "F.Cu") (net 17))
 (segment (start 175.6625 110.9) (end 175.7125 110.85) (width 0.2) (layer "F.Cu") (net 17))
 (via (at 165.8 110.9) (size 0.6) (drill 0.3) (layers "F.Cu" "B.Cu") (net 17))
 (via (at 160.185455 110.897523) (size 0.6) (drill 0.3) (layers "F.Cu" "B.Cu") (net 17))
 (segment (start 160.185455 110.897523) (end 160.187932 110.9) (width 0.2) (layer "B.Cu") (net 17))
 (segment (start 160.187932 110.9) (end 165.8 110.9) (width 0.2) (layer "B.Cu") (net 17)))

